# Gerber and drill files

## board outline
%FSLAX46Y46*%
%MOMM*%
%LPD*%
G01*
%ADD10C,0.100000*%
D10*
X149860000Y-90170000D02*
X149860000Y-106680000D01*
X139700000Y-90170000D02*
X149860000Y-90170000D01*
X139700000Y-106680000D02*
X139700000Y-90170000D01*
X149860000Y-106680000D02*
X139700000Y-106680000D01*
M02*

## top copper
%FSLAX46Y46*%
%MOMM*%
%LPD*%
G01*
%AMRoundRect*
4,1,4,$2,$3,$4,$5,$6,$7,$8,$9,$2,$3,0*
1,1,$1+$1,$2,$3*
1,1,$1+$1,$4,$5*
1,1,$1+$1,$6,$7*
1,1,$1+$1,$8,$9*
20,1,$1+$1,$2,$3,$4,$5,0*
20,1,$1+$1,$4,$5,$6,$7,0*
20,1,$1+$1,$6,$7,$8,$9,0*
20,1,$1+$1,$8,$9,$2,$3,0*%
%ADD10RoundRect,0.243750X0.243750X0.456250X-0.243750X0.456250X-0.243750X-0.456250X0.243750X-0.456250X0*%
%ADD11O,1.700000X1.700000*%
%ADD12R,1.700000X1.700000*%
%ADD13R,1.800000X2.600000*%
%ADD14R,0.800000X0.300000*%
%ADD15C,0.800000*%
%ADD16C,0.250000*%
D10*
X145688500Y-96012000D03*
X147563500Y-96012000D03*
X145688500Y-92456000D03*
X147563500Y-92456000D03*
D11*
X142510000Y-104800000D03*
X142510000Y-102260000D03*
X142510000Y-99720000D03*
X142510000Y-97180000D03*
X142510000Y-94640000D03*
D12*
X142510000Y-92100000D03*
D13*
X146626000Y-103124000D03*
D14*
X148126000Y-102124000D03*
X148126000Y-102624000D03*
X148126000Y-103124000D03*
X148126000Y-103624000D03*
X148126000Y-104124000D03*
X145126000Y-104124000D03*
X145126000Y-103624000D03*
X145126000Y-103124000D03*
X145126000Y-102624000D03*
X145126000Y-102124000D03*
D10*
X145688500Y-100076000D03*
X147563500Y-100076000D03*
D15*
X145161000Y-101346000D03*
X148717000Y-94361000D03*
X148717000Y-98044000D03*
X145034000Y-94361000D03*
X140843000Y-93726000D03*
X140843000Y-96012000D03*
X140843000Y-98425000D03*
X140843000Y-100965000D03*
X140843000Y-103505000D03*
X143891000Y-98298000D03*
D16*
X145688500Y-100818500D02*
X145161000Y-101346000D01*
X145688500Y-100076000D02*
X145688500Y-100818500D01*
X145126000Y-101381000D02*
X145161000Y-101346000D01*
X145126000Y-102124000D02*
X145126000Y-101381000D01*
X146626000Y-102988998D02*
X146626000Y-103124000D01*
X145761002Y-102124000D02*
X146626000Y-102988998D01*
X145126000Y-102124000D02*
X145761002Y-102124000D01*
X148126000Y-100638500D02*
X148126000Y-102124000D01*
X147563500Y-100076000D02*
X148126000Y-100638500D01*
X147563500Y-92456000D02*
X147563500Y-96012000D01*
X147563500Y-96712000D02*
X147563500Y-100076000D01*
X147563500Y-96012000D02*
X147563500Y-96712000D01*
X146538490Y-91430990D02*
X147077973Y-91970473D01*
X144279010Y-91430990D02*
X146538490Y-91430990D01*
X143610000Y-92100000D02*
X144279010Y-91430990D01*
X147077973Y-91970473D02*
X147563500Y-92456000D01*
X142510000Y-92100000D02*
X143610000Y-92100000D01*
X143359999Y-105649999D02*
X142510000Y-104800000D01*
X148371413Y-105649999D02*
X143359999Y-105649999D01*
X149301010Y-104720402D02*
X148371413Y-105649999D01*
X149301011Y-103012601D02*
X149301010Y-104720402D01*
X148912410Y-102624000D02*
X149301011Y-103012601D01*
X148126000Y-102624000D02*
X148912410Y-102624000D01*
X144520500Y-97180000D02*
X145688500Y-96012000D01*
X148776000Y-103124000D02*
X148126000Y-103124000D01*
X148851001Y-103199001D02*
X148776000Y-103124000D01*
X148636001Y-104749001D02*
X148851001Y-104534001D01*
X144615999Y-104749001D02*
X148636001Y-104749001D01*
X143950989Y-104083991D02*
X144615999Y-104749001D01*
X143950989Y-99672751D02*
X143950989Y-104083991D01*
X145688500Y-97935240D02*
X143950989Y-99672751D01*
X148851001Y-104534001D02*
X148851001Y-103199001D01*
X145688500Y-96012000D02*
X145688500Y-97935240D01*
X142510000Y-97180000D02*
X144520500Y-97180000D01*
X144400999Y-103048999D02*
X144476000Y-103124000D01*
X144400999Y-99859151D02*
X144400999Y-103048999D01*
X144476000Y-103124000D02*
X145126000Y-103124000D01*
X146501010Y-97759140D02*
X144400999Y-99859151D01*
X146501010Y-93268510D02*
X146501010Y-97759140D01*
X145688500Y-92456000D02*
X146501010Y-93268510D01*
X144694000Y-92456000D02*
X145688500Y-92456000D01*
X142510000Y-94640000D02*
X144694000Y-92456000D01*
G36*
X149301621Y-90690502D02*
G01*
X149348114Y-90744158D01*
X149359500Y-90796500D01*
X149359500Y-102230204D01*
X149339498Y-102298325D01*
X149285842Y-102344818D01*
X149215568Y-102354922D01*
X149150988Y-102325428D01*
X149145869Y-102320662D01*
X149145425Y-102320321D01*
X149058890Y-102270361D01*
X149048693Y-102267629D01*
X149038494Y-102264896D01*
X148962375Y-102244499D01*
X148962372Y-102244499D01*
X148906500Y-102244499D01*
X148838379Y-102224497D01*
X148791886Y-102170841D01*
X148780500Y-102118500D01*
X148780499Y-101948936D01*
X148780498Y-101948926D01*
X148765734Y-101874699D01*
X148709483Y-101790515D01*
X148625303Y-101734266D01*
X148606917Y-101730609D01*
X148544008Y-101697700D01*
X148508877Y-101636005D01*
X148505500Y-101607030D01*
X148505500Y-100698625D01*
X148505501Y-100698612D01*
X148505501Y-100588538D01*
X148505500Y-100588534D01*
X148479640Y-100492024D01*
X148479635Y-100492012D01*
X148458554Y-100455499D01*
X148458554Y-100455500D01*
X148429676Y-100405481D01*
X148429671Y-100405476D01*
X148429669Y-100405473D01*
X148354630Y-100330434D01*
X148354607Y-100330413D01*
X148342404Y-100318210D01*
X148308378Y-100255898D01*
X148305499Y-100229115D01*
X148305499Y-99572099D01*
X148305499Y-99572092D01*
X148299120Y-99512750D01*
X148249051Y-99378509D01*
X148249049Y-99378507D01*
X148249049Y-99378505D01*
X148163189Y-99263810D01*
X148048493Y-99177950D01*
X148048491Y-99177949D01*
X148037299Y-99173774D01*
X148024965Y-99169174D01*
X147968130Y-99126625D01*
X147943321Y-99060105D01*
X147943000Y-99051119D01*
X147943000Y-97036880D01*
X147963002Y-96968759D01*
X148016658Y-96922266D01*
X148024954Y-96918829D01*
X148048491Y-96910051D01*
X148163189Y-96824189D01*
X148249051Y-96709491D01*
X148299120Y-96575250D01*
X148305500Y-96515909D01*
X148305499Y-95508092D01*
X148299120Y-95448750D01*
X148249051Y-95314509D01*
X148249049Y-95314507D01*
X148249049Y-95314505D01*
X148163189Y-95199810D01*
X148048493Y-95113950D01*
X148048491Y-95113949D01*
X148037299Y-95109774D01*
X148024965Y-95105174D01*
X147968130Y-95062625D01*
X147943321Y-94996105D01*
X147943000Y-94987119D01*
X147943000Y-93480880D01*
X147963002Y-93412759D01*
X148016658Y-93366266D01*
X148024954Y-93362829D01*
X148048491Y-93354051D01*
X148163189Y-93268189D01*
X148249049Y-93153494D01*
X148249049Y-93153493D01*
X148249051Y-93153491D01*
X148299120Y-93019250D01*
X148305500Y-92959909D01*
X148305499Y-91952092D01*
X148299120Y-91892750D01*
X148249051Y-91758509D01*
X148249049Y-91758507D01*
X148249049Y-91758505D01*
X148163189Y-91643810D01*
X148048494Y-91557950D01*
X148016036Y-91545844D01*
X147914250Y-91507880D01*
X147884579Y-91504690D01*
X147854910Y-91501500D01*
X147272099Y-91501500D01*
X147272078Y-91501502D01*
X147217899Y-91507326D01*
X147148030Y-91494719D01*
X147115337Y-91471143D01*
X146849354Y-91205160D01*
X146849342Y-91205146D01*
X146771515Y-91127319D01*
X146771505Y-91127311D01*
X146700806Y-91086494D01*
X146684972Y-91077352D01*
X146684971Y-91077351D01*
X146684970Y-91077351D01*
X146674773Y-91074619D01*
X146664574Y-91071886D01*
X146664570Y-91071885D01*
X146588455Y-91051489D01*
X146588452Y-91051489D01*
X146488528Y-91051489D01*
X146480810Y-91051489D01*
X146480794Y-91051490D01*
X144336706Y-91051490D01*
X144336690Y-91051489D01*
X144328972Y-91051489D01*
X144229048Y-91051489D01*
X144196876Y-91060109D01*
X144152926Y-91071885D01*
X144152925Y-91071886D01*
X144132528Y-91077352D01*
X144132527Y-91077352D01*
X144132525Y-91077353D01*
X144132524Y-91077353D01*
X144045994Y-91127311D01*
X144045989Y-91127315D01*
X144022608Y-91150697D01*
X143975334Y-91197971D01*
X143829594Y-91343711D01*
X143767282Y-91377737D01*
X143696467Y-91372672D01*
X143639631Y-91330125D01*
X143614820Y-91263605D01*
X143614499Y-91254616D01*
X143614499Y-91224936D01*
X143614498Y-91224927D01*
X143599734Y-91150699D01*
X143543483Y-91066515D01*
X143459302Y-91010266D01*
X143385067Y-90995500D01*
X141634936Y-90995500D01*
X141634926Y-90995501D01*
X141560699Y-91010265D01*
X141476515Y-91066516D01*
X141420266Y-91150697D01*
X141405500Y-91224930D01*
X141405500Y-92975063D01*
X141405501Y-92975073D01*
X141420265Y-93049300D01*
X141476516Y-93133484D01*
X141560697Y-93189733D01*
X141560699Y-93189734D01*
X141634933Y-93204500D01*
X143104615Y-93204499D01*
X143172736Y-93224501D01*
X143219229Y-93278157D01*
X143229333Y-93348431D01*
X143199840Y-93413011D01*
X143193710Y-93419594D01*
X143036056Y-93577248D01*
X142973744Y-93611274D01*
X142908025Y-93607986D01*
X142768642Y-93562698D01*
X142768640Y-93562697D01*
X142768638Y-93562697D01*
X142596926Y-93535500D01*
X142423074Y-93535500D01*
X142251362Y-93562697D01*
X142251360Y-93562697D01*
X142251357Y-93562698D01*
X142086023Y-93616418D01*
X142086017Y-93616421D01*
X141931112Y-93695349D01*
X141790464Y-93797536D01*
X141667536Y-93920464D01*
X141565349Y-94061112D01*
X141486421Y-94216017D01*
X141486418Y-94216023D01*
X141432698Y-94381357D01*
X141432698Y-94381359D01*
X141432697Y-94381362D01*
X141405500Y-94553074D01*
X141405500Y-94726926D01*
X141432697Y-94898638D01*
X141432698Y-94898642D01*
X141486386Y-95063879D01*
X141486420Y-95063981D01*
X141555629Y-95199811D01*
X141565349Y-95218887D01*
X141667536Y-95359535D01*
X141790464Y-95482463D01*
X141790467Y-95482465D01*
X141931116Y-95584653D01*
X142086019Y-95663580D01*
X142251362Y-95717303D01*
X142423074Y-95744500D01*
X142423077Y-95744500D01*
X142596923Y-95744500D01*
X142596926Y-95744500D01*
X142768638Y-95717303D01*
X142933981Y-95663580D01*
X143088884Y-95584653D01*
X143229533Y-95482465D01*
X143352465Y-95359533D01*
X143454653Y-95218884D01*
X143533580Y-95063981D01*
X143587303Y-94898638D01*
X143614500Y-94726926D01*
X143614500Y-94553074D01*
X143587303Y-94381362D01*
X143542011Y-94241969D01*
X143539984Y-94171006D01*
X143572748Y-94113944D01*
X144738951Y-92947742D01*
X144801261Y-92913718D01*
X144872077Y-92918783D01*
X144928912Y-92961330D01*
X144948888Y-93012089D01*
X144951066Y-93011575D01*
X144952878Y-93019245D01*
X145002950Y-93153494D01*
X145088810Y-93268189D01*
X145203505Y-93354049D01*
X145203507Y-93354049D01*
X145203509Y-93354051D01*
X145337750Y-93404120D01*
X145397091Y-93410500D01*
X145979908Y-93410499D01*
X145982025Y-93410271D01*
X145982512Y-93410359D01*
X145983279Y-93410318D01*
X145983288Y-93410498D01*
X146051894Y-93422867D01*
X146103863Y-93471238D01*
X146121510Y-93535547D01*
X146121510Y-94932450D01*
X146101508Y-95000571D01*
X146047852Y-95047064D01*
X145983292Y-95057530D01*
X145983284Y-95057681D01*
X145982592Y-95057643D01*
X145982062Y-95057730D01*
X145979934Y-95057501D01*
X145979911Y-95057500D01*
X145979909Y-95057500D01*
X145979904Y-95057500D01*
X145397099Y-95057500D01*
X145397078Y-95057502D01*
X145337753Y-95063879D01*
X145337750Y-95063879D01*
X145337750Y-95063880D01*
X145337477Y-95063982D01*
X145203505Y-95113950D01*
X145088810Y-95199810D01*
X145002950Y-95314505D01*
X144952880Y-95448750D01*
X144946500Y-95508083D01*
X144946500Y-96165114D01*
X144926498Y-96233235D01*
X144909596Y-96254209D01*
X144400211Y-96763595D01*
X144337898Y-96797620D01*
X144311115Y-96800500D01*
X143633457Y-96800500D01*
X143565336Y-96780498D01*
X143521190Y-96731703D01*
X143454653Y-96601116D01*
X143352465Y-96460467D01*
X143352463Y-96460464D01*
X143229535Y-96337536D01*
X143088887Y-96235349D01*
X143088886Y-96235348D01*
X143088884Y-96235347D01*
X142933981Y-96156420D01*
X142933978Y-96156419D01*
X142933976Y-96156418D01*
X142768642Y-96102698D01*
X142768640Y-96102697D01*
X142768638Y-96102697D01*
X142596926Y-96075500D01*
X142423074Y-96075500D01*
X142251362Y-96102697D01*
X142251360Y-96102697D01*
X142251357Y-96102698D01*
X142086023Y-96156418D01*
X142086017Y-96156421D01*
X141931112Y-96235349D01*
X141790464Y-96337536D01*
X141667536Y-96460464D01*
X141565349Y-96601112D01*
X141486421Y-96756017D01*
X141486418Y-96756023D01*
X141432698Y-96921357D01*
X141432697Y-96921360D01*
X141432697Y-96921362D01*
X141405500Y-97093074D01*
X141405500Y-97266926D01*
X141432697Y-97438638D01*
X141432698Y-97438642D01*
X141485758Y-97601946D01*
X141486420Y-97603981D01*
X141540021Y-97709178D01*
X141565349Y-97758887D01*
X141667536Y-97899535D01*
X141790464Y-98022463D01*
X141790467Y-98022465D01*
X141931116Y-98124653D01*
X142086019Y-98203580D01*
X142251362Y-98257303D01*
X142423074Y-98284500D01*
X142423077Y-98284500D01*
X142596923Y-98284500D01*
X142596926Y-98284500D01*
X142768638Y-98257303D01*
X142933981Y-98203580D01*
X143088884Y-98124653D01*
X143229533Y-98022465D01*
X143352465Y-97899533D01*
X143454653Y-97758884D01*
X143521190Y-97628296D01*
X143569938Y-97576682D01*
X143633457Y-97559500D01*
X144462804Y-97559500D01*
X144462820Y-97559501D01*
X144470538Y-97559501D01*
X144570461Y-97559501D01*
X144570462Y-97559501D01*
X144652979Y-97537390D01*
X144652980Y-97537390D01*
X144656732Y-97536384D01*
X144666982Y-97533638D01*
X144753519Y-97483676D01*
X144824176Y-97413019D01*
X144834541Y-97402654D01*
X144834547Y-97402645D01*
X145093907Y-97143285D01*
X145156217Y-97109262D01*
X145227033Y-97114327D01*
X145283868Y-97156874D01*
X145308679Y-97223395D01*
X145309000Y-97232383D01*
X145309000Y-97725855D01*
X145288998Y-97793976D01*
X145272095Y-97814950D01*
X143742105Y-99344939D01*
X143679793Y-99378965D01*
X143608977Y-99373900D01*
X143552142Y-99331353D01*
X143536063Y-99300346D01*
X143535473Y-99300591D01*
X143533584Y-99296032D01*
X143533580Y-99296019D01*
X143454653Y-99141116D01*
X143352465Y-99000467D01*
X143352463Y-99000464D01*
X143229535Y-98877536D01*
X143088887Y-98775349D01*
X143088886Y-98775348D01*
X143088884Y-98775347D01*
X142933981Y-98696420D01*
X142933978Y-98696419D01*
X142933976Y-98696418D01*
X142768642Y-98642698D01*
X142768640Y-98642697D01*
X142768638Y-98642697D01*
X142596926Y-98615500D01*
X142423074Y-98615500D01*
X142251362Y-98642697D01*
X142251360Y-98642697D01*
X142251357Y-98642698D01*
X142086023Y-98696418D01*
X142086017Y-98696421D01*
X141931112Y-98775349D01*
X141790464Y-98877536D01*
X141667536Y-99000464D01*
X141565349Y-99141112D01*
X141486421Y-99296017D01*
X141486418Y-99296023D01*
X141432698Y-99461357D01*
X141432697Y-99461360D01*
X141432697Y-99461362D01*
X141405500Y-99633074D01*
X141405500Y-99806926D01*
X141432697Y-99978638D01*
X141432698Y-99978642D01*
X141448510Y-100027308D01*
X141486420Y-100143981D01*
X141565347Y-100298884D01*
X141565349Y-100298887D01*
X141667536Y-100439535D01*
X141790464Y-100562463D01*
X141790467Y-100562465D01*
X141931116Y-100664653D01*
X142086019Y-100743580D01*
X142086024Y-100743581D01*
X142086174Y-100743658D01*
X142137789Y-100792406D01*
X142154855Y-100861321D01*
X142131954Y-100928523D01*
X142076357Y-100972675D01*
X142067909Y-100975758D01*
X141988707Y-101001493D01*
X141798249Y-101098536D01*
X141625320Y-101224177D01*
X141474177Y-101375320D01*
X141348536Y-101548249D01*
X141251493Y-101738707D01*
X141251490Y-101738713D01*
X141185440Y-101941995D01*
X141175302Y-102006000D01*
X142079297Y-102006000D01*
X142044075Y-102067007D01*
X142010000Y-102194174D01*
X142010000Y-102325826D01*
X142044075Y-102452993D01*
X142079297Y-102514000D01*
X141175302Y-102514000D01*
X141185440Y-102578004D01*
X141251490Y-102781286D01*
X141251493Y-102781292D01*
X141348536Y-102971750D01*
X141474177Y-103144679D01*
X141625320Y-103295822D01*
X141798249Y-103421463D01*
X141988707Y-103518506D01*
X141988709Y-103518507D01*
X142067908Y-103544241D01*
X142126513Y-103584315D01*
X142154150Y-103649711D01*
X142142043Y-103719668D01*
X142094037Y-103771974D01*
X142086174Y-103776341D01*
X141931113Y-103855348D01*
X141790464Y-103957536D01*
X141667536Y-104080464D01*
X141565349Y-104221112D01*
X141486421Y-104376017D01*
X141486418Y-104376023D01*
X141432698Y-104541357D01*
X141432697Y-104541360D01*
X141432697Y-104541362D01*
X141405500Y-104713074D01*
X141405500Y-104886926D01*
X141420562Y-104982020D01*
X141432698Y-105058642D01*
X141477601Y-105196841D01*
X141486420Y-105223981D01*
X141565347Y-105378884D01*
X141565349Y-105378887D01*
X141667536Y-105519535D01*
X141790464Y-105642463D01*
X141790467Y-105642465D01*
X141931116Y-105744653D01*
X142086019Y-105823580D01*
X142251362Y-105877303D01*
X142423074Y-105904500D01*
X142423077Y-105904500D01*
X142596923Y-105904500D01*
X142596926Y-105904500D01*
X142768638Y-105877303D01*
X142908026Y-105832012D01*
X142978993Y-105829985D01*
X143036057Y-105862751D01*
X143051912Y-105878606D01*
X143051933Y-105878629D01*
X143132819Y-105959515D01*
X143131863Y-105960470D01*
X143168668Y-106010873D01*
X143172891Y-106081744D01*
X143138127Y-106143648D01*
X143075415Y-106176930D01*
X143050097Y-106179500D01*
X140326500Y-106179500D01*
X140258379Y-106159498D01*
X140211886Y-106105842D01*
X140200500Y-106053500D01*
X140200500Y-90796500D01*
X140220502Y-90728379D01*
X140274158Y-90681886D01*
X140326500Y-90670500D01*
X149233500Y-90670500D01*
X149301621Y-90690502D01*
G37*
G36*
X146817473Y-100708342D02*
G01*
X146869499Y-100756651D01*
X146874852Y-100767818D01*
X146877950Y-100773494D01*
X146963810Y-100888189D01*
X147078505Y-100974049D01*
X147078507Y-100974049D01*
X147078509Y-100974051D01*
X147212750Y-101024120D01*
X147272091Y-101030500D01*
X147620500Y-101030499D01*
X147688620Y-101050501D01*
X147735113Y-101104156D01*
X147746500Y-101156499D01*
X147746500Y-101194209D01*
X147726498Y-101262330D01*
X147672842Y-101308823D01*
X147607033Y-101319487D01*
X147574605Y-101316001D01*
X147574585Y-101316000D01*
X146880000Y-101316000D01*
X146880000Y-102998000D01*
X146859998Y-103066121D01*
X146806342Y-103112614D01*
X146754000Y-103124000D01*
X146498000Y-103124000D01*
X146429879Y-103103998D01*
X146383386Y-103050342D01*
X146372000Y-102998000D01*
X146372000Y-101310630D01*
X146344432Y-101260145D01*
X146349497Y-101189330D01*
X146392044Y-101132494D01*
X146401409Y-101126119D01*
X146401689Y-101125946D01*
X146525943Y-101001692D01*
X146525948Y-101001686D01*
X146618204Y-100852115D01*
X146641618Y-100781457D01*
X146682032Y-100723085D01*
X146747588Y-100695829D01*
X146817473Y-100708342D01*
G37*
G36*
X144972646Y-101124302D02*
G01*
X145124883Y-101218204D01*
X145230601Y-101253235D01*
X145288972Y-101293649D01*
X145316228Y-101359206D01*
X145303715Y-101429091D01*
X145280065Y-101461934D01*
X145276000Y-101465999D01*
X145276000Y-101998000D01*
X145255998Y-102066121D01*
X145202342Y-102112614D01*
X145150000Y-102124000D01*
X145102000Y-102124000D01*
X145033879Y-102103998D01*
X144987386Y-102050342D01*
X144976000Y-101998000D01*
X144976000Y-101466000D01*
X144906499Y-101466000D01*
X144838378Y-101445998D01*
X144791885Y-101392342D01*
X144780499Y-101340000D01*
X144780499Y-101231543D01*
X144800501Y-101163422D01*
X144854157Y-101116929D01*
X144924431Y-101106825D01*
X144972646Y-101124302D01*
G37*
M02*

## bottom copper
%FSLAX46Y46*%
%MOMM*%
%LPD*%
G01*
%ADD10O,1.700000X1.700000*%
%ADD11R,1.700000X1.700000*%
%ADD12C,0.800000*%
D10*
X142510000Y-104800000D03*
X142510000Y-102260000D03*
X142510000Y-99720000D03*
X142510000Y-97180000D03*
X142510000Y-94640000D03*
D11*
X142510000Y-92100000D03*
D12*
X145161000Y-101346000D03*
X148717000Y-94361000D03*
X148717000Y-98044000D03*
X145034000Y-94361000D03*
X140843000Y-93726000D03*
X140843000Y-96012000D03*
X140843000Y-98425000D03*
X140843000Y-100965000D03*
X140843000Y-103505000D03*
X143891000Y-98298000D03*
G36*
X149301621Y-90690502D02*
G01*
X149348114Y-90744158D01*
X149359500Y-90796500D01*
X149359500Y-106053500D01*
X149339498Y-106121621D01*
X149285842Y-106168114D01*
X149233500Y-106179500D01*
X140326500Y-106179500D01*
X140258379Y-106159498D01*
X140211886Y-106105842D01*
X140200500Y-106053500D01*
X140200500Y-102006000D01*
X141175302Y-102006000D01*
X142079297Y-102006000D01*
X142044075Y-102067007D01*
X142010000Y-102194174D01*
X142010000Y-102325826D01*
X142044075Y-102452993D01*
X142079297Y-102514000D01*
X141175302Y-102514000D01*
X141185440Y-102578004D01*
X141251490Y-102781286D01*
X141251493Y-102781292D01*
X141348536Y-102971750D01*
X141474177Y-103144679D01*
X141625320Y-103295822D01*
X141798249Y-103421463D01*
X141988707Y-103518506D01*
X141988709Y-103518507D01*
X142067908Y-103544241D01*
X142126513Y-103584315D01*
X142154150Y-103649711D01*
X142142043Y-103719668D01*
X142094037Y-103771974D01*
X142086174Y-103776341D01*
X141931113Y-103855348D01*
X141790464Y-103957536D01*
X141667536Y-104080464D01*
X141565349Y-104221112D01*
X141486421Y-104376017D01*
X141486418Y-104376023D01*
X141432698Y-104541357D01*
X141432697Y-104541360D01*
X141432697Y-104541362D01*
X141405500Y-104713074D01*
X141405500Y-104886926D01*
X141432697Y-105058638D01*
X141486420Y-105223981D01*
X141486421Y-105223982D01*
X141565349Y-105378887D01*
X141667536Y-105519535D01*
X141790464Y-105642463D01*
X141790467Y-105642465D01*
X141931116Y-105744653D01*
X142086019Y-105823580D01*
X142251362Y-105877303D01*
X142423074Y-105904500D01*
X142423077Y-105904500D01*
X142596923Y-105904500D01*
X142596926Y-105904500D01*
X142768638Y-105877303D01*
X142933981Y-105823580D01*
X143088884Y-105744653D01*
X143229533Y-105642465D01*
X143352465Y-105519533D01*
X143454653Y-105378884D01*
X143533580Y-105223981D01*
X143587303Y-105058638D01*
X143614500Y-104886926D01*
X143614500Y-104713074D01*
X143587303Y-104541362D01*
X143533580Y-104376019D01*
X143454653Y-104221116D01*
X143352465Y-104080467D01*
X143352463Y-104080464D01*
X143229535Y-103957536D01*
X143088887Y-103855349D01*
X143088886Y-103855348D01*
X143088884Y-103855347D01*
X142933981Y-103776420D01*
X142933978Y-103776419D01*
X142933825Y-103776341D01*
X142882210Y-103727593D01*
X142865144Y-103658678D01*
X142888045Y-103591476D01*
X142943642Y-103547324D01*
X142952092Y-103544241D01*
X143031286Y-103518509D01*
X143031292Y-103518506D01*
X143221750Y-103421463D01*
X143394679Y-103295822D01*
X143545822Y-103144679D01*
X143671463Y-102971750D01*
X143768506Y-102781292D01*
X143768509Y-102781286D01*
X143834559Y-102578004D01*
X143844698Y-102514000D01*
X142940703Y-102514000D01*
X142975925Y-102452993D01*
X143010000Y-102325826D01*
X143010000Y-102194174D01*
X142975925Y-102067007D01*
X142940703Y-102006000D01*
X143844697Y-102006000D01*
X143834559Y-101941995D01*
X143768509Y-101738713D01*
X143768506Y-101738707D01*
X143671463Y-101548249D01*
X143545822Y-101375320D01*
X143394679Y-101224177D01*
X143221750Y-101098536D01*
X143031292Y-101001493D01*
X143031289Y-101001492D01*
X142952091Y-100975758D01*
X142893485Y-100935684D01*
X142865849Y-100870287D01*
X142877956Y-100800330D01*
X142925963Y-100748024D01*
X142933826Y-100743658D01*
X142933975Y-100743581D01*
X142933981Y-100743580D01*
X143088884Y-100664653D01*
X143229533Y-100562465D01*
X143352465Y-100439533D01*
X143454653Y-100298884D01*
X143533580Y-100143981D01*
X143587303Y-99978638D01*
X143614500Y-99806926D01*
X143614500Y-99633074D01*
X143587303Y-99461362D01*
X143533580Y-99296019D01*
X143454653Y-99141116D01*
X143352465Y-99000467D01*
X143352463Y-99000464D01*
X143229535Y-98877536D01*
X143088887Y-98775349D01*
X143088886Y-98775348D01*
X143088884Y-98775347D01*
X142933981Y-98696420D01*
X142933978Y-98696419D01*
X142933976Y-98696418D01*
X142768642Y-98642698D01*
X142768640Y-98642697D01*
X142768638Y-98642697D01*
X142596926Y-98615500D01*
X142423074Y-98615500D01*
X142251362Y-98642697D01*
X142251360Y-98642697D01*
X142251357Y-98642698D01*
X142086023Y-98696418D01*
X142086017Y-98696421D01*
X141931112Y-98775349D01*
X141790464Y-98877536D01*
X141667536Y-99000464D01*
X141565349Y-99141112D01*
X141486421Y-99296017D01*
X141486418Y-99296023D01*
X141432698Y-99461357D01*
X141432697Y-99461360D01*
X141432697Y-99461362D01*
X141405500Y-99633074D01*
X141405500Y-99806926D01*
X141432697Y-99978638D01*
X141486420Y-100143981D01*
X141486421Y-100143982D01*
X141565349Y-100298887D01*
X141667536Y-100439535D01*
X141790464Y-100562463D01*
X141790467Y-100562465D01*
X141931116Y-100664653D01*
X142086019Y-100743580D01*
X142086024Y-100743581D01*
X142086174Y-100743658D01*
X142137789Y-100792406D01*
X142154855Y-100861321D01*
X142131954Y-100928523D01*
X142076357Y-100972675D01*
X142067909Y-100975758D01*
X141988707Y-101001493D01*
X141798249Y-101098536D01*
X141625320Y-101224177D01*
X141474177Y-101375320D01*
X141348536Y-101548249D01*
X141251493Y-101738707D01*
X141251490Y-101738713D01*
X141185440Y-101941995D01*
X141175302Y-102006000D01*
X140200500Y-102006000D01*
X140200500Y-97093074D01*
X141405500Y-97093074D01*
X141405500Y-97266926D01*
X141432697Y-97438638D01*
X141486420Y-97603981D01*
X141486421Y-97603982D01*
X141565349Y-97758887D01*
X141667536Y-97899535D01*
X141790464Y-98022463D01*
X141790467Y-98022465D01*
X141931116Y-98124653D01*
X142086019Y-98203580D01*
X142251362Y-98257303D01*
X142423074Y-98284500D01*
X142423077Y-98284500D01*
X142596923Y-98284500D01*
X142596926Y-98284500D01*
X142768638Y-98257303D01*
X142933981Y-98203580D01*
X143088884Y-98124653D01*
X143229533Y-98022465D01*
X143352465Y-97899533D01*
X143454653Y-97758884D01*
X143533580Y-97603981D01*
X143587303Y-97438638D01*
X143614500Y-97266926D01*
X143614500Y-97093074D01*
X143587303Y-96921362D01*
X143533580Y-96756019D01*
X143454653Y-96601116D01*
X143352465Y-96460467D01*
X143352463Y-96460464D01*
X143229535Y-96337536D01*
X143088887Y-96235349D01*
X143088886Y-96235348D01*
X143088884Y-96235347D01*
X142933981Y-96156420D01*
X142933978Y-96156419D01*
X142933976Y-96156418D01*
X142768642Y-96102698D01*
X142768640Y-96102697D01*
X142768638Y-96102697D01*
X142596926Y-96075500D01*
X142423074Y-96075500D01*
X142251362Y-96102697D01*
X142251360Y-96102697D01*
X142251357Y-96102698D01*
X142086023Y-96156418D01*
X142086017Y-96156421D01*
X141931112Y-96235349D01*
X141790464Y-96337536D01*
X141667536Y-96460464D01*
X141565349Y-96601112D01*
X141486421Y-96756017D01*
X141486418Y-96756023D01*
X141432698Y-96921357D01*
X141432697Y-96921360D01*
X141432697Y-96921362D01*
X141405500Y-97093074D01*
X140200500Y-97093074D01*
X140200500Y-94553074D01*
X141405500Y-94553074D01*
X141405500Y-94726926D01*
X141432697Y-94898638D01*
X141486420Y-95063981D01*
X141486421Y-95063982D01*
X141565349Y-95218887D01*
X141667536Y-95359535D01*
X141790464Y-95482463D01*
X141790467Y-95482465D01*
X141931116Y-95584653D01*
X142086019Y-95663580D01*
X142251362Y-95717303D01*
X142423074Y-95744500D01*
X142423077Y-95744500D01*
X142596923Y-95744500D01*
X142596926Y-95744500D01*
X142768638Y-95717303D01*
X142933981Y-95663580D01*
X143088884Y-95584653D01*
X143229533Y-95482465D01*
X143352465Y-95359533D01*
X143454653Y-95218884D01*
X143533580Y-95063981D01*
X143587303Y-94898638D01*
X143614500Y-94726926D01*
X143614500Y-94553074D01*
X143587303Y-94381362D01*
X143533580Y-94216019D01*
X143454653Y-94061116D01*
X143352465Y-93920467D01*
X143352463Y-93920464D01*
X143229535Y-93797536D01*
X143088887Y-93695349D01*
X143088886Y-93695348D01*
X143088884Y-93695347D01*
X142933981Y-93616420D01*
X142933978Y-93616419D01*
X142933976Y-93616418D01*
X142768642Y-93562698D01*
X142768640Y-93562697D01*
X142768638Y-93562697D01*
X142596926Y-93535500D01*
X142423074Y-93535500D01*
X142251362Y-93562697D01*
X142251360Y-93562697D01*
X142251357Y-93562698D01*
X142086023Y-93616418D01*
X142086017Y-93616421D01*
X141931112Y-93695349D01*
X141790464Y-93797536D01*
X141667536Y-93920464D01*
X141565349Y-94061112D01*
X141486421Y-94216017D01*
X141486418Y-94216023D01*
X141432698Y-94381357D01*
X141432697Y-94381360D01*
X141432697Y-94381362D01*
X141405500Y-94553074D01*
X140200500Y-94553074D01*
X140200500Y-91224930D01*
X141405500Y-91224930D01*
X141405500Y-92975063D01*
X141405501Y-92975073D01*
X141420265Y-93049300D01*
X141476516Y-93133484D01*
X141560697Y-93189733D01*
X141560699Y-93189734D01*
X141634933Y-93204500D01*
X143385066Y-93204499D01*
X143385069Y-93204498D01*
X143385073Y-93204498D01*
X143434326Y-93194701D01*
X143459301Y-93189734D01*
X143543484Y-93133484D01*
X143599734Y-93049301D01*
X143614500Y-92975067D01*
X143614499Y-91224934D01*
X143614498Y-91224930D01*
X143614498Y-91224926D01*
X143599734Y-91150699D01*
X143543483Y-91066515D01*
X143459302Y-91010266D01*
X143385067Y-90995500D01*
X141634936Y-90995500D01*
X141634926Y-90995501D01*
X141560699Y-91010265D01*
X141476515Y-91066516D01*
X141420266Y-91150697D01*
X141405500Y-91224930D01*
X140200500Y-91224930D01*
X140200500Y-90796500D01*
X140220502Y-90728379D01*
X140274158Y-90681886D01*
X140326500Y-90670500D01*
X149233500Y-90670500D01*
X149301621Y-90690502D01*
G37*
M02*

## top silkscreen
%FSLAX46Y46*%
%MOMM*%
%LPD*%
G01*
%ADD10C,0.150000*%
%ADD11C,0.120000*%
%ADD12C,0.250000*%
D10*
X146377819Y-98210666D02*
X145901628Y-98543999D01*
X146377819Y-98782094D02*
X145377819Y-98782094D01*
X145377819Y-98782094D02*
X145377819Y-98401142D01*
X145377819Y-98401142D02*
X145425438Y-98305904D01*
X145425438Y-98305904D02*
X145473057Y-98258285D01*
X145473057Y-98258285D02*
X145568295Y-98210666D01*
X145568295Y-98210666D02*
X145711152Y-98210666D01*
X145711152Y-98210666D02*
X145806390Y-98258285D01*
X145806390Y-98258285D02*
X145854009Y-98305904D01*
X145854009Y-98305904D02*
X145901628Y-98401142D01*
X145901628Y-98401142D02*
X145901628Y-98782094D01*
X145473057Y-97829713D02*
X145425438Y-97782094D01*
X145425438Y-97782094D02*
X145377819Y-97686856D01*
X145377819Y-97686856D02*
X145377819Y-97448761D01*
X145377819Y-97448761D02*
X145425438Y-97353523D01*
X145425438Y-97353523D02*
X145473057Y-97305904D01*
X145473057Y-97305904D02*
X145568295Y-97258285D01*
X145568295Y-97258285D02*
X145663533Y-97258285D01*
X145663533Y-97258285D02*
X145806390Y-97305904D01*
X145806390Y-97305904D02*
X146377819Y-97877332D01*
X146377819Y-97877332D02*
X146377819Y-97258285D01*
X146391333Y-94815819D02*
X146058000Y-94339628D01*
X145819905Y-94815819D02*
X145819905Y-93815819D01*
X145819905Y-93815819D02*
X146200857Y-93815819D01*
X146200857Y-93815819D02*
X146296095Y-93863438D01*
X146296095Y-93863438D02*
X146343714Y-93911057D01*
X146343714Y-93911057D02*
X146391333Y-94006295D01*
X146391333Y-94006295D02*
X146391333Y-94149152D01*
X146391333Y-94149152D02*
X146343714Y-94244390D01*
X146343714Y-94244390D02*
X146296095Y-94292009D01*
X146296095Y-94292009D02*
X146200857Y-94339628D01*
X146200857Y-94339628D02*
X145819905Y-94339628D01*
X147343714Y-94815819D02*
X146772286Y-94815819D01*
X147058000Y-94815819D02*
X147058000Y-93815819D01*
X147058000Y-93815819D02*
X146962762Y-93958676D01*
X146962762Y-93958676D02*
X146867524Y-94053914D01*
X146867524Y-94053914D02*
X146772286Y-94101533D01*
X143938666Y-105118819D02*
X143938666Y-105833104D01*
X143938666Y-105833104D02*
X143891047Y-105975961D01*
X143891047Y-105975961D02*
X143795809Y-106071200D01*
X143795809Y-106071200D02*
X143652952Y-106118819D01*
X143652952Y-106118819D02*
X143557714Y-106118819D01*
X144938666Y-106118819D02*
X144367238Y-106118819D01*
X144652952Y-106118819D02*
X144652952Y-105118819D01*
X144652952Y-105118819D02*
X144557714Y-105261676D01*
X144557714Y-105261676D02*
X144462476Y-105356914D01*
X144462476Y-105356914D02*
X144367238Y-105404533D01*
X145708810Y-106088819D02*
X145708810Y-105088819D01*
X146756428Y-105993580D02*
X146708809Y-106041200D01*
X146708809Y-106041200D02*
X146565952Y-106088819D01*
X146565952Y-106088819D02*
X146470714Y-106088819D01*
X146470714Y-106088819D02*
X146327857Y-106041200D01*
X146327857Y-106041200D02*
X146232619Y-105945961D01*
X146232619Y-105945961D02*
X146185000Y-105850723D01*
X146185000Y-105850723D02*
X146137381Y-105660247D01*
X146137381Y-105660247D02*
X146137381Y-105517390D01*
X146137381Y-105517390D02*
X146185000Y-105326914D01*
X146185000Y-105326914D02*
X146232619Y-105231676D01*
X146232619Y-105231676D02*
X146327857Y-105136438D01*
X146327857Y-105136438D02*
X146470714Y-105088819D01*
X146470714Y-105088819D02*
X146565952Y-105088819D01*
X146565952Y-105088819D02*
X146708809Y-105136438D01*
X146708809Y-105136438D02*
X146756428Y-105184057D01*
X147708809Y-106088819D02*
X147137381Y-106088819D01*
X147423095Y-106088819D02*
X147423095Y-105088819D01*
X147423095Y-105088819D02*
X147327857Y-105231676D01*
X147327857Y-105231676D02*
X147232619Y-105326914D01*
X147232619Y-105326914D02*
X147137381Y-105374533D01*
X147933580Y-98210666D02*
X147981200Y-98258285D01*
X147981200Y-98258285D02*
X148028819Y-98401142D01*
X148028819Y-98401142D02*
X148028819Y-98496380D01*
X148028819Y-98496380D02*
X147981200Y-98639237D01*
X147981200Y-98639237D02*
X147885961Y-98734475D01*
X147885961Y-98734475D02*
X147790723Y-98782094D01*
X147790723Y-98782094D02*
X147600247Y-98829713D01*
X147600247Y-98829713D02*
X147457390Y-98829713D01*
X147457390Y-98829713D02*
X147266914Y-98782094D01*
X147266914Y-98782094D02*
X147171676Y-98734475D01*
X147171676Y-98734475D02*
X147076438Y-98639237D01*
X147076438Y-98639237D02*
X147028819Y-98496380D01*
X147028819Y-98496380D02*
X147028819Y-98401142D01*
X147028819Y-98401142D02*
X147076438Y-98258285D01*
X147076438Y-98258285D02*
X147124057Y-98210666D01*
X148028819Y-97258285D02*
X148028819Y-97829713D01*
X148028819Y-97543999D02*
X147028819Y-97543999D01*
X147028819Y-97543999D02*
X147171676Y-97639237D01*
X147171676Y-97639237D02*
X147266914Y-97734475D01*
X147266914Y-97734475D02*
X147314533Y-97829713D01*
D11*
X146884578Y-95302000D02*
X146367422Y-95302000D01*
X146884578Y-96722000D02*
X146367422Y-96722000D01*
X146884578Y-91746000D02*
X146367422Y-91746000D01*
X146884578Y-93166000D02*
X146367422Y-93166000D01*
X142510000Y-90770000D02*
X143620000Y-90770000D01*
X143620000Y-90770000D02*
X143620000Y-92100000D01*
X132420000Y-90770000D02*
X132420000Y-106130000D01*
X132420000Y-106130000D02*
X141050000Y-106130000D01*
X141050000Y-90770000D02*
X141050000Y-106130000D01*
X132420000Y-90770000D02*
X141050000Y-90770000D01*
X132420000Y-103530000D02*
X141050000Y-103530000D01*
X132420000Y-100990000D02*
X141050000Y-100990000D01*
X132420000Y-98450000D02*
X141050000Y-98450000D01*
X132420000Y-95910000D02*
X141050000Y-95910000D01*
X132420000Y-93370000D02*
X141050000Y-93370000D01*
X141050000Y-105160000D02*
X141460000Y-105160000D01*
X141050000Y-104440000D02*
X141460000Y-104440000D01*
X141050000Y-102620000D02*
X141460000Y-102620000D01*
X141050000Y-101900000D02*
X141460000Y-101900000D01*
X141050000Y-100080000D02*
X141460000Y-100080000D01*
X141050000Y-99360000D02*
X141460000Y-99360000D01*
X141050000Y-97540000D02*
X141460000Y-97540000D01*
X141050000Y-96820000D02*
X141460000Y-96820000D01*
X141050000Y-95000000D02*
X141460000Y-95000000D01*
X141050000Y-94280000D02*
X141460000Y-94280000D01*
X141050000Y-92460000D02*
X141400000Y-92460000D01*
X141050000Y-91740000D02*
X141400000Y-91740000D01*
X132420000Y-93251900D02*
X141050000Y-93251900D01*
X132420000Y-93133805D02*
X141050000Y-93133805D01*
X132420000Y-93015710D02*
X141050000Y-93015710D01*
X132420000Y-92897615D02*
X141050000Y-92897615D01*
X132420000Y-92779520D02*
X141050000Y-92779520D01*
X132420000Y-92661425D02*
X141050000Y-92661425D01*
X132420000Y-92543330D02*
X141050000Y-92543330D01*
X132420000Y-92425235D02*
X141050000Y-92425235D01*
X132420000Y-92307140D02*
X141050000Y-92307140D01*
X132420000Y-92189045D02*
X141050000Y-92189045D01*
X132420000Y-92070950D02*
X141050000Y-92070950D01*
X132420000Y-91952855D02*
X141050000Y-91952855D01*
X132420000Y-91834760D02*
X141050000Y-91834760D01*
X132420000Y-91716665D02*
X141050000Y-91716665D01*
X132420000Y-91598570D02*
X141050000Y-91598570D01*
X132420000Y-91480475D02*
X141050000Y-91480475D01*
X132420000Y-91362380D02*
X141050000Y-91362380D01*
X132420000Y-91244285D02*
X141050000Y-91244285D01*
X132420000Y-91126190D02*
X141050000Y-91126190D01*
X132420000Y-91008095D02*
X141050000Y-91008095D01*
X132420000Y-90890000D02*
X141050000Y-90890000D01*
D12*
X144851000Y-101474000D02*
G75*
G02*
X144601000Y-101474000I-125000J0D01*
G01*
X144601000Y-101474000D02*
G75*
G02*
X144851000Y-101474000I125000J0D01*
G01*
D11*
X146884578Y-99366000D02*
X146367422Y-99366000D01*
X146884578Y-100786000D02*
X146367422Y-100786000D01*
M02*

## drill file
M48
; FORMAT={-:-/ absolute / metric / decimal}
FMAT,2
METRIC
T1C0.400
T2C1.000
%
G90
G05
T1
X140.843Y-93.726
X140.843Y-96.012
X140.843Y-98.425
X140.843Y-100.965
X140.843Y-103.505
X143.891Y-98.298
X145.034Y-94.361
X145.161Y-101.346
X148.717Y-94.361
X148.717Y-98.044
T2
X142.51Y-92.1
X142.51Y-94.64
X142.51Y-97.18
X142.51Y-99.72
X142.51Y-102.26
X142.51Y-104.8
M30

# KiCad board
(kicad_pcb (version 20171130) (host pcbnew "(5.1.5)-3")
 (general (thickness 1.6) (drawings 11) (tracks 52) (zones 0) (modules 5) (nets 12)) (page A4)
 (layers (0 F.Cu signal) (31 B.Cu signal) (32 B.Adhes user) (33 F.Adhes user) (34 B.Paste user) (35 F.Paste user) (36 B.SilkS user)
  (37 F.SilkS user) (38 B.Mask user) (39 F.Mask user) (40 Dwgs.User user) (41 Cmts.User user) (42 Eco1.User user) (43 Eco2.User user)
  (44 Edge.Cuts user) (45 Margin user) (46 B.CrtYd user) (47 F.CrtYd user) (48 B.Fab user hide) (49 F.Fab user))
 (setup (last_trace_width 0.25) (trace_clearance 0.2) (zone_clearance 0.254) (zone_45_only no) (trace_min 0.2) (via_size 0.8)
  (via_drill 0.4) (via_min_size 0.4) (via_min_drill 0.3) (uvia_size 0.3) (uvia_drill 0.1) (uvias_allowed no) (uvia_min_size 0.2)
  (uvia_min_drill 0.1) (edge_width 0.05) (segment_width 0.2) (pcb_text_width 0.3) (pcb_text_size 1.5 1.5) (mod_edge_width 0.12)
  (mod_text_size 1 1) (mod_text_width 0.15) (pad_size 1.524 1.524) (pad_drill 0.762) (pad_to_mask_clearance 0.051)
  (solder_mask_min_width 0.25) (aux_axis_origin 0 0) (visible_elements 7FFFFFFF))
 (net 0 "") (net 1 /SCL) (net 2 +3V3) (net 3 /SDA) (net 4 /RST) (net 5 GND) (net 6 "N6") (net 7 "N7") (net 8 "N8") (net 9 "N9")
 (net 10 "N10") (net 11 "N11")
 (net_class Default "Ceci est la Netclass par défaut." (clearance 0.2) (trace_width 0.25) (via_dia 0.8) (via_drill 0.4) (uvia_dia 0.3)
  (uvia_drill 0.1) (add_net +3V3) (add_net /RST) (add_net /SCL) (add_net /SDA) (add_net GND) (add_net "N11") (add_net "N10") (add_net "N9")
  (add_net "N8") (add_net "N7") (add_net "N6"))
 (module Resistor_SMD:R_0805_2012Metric (layer F.Cu) (at 146.626 96.012 180)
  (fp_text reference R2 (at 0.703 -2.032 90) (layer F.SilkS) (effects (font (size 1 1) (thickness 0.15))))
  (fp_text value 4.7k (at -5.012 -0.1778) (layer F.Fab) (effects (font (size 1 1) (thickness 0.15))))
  (fp_line (start -0.258578 0.71) (end 0.258578 0.71) (layer F.SilkS) (width 0.12))
  (fp_line (start -0.258578 -0.71) (end 0.258578 -0.71) (layer F.SilkS) (width 0.12))
  (pad 2 smd roundrect (at 0.9375 0 180) (size 0.975 1.4) (layers F.Cu F.Paste F.Mask) (roundrect_rratio 0.25) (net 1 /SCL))
  (pad 1 smd roundrect (at -0.9375 0 180) (size 0.975 1.4) (layers F.Cu F.Paste F.Mask) (roundrect_rratio 0.25) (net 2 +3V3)))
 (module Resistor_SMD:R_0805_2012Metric (layer F.Cu) (at 146.626 92.456 180)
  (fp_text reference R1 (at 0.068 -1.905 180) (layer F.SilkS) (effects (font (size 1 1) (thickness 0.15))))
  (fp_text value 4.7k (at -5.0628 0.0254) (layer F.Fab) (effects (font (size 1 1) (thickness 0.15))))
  (fp_line (start -0.258578 0.71) (end 0.258578 0.71) (layer F.SilkS) (width 0.12))
  (fp_line (start -0.258578 -0.71) (end 0.258578 -0.71) (layer F.SilkS) (width 0.12))
  (pad 2 smd roundrect (at 0.9375 0 180) (size 0.975 1.4) (layers F.Cu F.Paste F.Mask) (roundrect_rratio 0.25) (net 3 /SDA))
  (pad 1 smd roundrect (at -0.9375 0 180) (size 0.975 1.4) (layers F.Cu F.Paste F.Mask) (roundrect_rratio 0.25) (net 2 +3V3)))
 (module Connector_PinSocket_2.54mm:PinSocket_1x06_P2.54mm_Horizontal (layer F.Cu) (at 142.51 92.1)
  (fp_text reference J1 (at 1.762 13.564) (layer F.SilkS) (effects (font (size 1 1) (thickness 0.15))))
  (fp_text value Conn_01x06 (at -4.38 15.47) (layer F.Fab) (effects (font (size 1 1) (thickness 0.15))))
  (fp_line (start 0 -1.33) (end 1.11 -1.33) (layer F.SilkS) (width 0.12))
  (fp_line (start 1.11 -1.33) (end 1.11 0) (layer F.SilkS) (width 0.12))
  (fp_line (start -10.09 -1.33) (end -10.09 14.03) (layer F.SilkS) (width 0.12))
  (fp_line (start -10.09 14.03) (end -1.46 14.03) (layer F.SilkS) (width 0.12))
  (fp_line (start -1.46 -1.33) (end -1.46 14.03) (layer F.SilkS) (width 0.12))
  (fp_line (start -10.09 -1.33) (end -1.46 -1.33) (layer F.SilkS) (width 0.12))
  (fp_line (start -10.09 11.43) (end -1.46 11.43) (layer F.SilkS) (width 0.12))
  (fp_line (start -10.09 8.89) (end -1.46 8.89) (layer F.SilkS) (width 0.12))
  (fp_line (start -10.09 6.35) (end -1.46 6.35) (layer F.SilkS) (width 0.12))
  (fp_line (start -10.09 3.81) (end -1.46 3.81) (layer F.SilkS) (width 0.12))
  (fp_line (start -10.09 1.27) (end -1.46 1.27) (layer F.SilkS) (width 0.12))
  (fp_line (start -1.46 13.06) (end -1.05 13.06) (layer F.SilkS) (width 0.12))
  (fp_line (start -1.46 12.34) (end -1.05 12.34) (layer F.SilkS) (width 0.12))
  (fp_line (start -1.46 10.52) (end -1.05 10.52) (layer F.SilkS) (width 0.12))
  (fp_line (start -1.46 9.8) (end -1.05 9.8) (layer F.SilkS) (width 0.12))
  (fp_line (start -1.46 7.98) (end -1.05 7.98) (layer F.SilkS) (width 0.12))
  (fp_line (start -1.46 7.26) (end -1.05 7.26) (layer F.SilkS) (width 0.12))
  (fp_line (start -1.46 5.44) (end -1.05 5.44) (layer F.SilkS) (width 0.12))
  (fp_line (start -1.46 4.72) (end -1.05 4.72) (layer F.SilkS) (width 0.12))
  (fp_line (start -1.46 2.9) (end -1.05 2.9) (layer F.SilkS) (width 0.12))
  (fp_line (start -1.46 2.18) (end -1.05 2.18) (layer F.SilkS) (width 0.12))
  (fp_line (start -1.46 0.36) (end -1.11 0.36) (layer F.SilkS) (width 0.12))
  (fp_line (start -1.46 -0.36) (end -1.11 -0.36) (layer F.SilkS) (width 0.12))
  (fp_line (start -10.09 1.1519) (end -1.46 1.1519) (layer F.SilkS) (width 0.12))
  (fp_line (start -10.09 1.033805) (end -1.46 1.033805) (layer F.SilkS) (width 0.12))
  (fp_line (start -10.09 0.91571) (end -1.46 0.91571) (layer F.SilkS) (width 0.12))
  (fp_line (start -10.09 0.797615) (end -1.46 0.797615) (layer F.SilkS) (width 0.12))
  (fp_line (start -10.09 0.67952) (end -1.46 0.67952) (layer F.SilkS) (width 0.12))
  (fp_line (start -10.09 0.561425) (end -1.46 0.561425) (layer F.SilkS) (width 0.12))
  (fp_line (start -10.09 0.44333) (end -1.46 0.44333) (layer F.SilkS) (width 0.12))
  (fp_line (start -10.09 0.325235) (end -1.46 0.325235) (layer F.SilkS) (width 0.12))
  (fp_line (start -10.09 0.20714) (end -1.46 0.20714) (layer F.SilkS) (width 0.12))
  (fp_line (start -10.09 0.089045) (end -1.46 0.089045) (layer F.SilkS) (width 0.12))
  (fp_line (start -10.09 -0.02905) (end -1.46 -0.02905) (layer F.SilkS) (width 0.12))
  (fp_line (start -10.09 -0.147145) (end -1.46 -0.147145) (layer F.SilkS) (width 0.12))
  (fp_line (start -10.09 -0.26524) (end -1.46 -0.26524) (layer F.SilkS) (width 0.12))
  (fp_line (start -10.09 -0.383335) (end -1.46 -0.383335) (layer F.SilkS) (width 0.12))
  (fp_line (start -10.09 -0.50143) (end -1.46 -0.50143) (layer F.SilkS) (width 0.12))
  (fp_line (start -10.09 -0.619525) (end -1.46 -0.619525) (layer F.SilkS) (width 0.12))
  (fp_line (start -10.09 -0.73762) (end -1.46 -0.73762) (layer F.SilkS) (width 0.12))
  (fp_line (start -10.09 -0.855715) (end -1.46 -0.855715) (layer F.SilkS) (width 0.12))
  (fp_line (start -10.09 -0.97381) (end -1.46 -0.97381) (layer F.SilkS) (width 0.12))
  (fp_line (start -10.09 -1.091905) (end -1.46 -1.091905) (layer F.SilkS) (width 0.12))
  (fp_line (start -10.09 -1.21) (end -1.46 -1.21) (layer F.SilkS) (width 0.12))
  (pad 6 thru_hole oval (at 0 12.7) (size 1.7 1.7) (drill 1) (layers *.Cu *.Mask) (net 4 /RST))
  (pad 5 thru_hole oval (at 0 10.16) (size 1.7 1.7) (drill 1) (layers *.Cu *.Mask) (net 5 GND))
  (pad 4 thru_hole oval (at 0 7.62) (size 1.7 1.7) (drill 1) (layers *.Cu *.Mask) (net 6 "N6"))
  (pad 3 thru_hole oval (at 0 5.08) (size 1.7 1.7) (drill 1) (layers *.Cu *.Mask) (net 1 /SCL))
  (pad 2 thru_hole oval (at 0 2.54) (size 1.7 1.7) (drill 1) (layers *.Cu *.Mask) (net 3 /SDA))
  (pad 1 thru_hole rect (at 0 0) (size 1.7 1.7) (drill 1) (layers *.Cu *.Mask) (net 2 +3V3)))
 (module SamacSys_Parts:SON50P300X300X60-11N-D (layer F.Cu) (at 146.626 103.124)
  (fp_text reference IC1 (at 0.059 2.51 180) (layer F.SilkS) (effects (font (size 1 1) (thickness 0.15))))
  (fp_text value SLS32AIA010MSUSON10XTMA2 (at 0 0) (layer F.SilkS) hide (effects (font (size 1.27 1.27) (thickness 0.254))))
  (fp_circle (center -1.9 -1.65) (end -1.9 -1.525) (layer F.SilkS) (width 0.25))
  (pad 11 smd rect (at 0 0) (size 1.8 2.6) (layers F.Cu F.Paste F.Mask) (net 5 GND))
  (pad 10 smd rect (at 1.5 -1 90) (size 0.3 0.8) (layers F.Cu F.Paste F.Mask) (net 2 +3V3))
  (pad 9 smd rect (at 1.5 -0.5 90) (size 0.3 0.8) (layers F.Cu F.Paste F.Mask) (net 4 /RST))
  (pad 8 smd rect (at 1.5 0 90) (size 0.3 0.8) (layers F.Cu F.Paste F.Mask) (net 1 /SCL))
  (pad 7 smd rect (at 1.5 0.5 90) (size 0.3 0.8) (layers F.Cu F.Paste F.Mask) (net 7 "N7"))
  (pad 6 smd rect (at 1.5 1 90) (size 0.3 0.8) (layers F.Cu F.Paste F.Mask) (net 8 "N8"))
  (pad 5 smd rect (at -1.5 1 90) (size 0.3 0.8) (layers F.Cu F.Paste F.Mask) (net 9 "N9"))
  (pad 4 smd rect (at -1.5 0.5 90) (size 0.3 0.8) (layers F.Cu F.Paste F.Mask) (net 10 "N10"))
  (pad 3 smd rect (at -1.5 0 90) (size 0.3 0.8) (layers F.Cu F.Paste F.Mask) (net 3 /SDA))
  (pad 2 smd rect (at -1.5 -0.5 90) (size 0.3 0.8) (layers F.Cu F.Paste F.Mask) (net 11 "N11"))
  (pad 1 smd rect (at -1.5 -1 90) (size 0.3 0.8) (layers F.Cu F.Paste F.Mask) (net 5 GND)))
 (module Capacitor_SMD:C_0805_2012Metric (layer F.Cu) (at 146.626 100.076 180)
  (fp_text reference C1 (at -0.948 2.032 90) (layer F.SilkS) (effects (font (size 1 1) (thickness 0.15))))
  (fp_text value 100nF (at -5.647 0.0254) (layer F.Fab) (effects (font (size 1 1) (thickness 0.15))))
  (fp_line (start -0.258578 0.71) (end 0.258578 0.71) (layer F.SilkS) (width 0.12))
  (fp_line (start -0.258578 -0.71) (end 0.258578 -0.71) (layer F.SilkS) (width 0.12))
  (pad 2 smd roundrect (at 0.9375 0 180) (size 0.975 1.4) (layers F.Cu F.Paste F.Mask) (roundrect_rratio 0.25) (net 5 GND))
  (pad 1 smd roundrect (at -0.9375 0 180) (size 0.975 1.4) (layers F.Cu F.Paste F.Mask) (roundrect_rratio 0.25) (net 2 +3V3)))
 (gr_line (start 149.86 90.17) (end 149.86 106.68) (layer Edge.Cuts) (width 0.1))
 (gr_line (start 139.7 90.17) (end 149.86 90.17) (layer Edge.Cuts) (width 0.1))
 (gr_line (start 139.7 106.68) (end 139.7 90.17) (layer Edge.Cuts) (width 0.1))
 (gr_line (start 149.86 106.68) (end 139.7 106.68) (layer Edge.Cuts) (width 0.1))
 (via (at 145.161 101.346) (size 0.8) (drill 0.4) (layers F.Cu B.Cu) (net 5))
 (via (at 148.717 94.361) (size 0.8) (drill 0.4) (layers F.Cu B.Cu) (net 5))
 (via (at 148.717 98.044) (size 0.8) (drill 0.4) (layers F.Cu B.Cu) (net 5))
 (via (at 145.034 94.361) (size 0.8) (drill 0.4) (layers F.Cu B.Cu) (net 5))
 (segment (start 145.6885 100.8185) (end 145.161 101.346) (width 0.25) (layer F.Cu) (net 5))
 (segment (start 145.6885 100.076) (end 145.6885 100.8185) (width 0.25) (layer F.Cu) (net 5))
 (segment (start 145.126 101.381) (end 145.161 101.346) (width 0.25) (layer F.Cu) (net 5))
 (segment (start 145.126 102.124) (end 145.126 101.381) (width 0.25) (layer F.Cu) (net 5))
 (segment (start 146.626 102.988998) (end 146.626 103.124) (width 0.25) (layer F.Cu) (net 5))
 (segment (start 145.761002 102.124) (end 146.626 102.988998) (width 0.25) (layer F.Cu) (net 5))
 (segment (start 145.126 102.124) (end 145.761002 102.124) (width 0.25) (layer F.Cu) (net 5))
 (via (at 140.843 93.726) (size 0.8) (drill 0.4) (layers F.Cu B.Cu) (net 5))
 (via (at 140.843 96.012) (size 0.8) (drill 0.4) (layers F.Cu B.Cu) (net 5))
 (via (at 140.843 98.425) (size 0.8) (drill 0.4) (layers F.Cu B.Cu) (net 5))
 (via (at 140.843 100.965) (size 0.8) (drill 0.4) (layers F.Cu B.Cu) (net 5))
 (via (at 140.843 103.505) (size 0.8) (drill 0.4) (layers F.Cu B.Cu) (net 5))
 (via (at 143.891 98.298) (size 0.8) (drill 0.4) (layers F.Cu B.Cu) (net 5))
 (segment (start 148.126 100.6385) (end 148.126 102.124) (width 0.25) (layer F.Cu) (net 2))
 (segment (start 147.5635 100.076) (end 148.126 100.6385) (width 0.25) (layer F.Cu) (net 2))
 (segment (start 147.5635 92.456) (end 147.5635 96.012) (width 0.25) (layer F.Cu) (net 2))
 (segment (start 147.5635 96.712) (end 147.5635 100.076) (width 0.25) (layer F.Cu) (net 2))
 (segment (start 147.5635 96.012) (end 147.5635 96.712) (width 0.25) (layer F.Cu) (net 2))
 (segment (start 146.53849 91.43099) (end 147.077973 91.970473) (width 0.25) (layer F.Cu) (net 2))
 (segment (start 144.27901 91.43099) (end 146.53849 91.43099) (width 0.25) (layer F.Cu) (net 2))
 (segment (start 143.61 92.1) (end 144.27901 91.43099) (width 0.25) (layer F.Cu) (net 2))
 (segment (start 147.077973 91.970473) (end 147.5635 92.456) (width 0.25) (layer F.Cu) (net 2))
 (segment (start 142.51 92.1) (end 143.61 92.1) (width 0.25) (layer F.Cu) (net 2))
 (segment (start 143.359999 105.649999) (end 142.51 104.8) (width 0.25) (layer F.Cu) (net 4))
 (segment (start 148.371413 105.649999) (end 143.359999 105.649999) (width 0.25) (layer F.Cu) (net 4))
 (segment (start 149.30101 104.720402) (end 148.371413 105.649999) (width 0.25) (layer F.Cu) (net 4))
 (segment (start 149.301011 103.012601) (end 149.30101 104.720402) (width 0.25) (layer F.Cu) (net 4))
 (segment (start 148.91241 102.624) (end 149.301011 103.012601) (width 0.25) (layer F.Cu) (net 4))
 (segment (start 148.126 102.624) (end 148.91241 102.624) (width 0.25) (layer F.Cu) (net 4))
 (segment (start 144.5205 97.18) (end 145.6885 96.012) (width 0.25) (layer F.Cu) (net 1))
 (segment (start 148.776 103.124) (end 148.126 103.124) (width 0.25) (layer F.Cu) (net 1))
 (segment (start 148.851001 103.199001) (end 148.776 103.124) (width 0.25) (layer F.Cu) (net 1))
 (segment (start 148.636001 104.749001) (end 148.851001 104.534001) (width 0.25) (layer F.Cu) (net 1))
 (segment (start 144.615999 104.749001) (end 148.636001 104.749001) (width 0.25) (layer F.Cu) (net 1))
 (segment (start 143.950989 104.083991) (end 144.615999 104.749001) (width 0.25) (layer F.Cu) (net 1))
 (segment (start 143.950989 99.672751) (end 143.950989 104.083991) (width 0.25) (layer F.Cu) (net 1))
 (segment (start 145.6885 97.93524) (end 143.950989 99.672751) (width 0.25) (layer F.Cu) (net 1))
 (segment (start 148.851001 104.534001) (end 148.851001 103.199001) (width 0.25) (layer F.Cu) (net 1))
 (segment (start 145.6885 96.012) (end 145.6885 97.93524) (width 0.25) (layer F.Cu) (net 1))
 (segment (start 142.51 97.18) (end 144.5205 97.18) (width 0.25) (layer F.Cu) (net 1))
 (segment (start 144.400999 103.048999) (end 144.476 103.124) (width 0.25) (layer F.Cu) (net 3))
 (segment (start 144.400999 99.859151) (end 144.400999 103.048999) (width 0.25) (layer F.Cu) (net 3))
 (segment (start 144.476 103.124) (end 145.126 103.124) (width 0.25) (layer F.Cu) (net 3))
 (segment (start 146.50101 97.75914) (end 144.400999 99.859151) (width 0.25) (layer F.Cu) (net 3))
 (segment (start 146.50101 93.26851) (end 146.50101 97.75914) (width 0.25) (layer F.Cu) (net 3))
 (segment (start 145.6885 92.456) (end 146.50101 93.26851) (width 0.25) (layer F.Cu) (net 3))
 (segment (start 144.694 92.456) (end 145.6885 92.456) (width 0.25) (layer F.Cu) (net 3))
 (segment (start 142.51 94.64) (end 144.694 92.456) (width 0.25) (layer F.Cu) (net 3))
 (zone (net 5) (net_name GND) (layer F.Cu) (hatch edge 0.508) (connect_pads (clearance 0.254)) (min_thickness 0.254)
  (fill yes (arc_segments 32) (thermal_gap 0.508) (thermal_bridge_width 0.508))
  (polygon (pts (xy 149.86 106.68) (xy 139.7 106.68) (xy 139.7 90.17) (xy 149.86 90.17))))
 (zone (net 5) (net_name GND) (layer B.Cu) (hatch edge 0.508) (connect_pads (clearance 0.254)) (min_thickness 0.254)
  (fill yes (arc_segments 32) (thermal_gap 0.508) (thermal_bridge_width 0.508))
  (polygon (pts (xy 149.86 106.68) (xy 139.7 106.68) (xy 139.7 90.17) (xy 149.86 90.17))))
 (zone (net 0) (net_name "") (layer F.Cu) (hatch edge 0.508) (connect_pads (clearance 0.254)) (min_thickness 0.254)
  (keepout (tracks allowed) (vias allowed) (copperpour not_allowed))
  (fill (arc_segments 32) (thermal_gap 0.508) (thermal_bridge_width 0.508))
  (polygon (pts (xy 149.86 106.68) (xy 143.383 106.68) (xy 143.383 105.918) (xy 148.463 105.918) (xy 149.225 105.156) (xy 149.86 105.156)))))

